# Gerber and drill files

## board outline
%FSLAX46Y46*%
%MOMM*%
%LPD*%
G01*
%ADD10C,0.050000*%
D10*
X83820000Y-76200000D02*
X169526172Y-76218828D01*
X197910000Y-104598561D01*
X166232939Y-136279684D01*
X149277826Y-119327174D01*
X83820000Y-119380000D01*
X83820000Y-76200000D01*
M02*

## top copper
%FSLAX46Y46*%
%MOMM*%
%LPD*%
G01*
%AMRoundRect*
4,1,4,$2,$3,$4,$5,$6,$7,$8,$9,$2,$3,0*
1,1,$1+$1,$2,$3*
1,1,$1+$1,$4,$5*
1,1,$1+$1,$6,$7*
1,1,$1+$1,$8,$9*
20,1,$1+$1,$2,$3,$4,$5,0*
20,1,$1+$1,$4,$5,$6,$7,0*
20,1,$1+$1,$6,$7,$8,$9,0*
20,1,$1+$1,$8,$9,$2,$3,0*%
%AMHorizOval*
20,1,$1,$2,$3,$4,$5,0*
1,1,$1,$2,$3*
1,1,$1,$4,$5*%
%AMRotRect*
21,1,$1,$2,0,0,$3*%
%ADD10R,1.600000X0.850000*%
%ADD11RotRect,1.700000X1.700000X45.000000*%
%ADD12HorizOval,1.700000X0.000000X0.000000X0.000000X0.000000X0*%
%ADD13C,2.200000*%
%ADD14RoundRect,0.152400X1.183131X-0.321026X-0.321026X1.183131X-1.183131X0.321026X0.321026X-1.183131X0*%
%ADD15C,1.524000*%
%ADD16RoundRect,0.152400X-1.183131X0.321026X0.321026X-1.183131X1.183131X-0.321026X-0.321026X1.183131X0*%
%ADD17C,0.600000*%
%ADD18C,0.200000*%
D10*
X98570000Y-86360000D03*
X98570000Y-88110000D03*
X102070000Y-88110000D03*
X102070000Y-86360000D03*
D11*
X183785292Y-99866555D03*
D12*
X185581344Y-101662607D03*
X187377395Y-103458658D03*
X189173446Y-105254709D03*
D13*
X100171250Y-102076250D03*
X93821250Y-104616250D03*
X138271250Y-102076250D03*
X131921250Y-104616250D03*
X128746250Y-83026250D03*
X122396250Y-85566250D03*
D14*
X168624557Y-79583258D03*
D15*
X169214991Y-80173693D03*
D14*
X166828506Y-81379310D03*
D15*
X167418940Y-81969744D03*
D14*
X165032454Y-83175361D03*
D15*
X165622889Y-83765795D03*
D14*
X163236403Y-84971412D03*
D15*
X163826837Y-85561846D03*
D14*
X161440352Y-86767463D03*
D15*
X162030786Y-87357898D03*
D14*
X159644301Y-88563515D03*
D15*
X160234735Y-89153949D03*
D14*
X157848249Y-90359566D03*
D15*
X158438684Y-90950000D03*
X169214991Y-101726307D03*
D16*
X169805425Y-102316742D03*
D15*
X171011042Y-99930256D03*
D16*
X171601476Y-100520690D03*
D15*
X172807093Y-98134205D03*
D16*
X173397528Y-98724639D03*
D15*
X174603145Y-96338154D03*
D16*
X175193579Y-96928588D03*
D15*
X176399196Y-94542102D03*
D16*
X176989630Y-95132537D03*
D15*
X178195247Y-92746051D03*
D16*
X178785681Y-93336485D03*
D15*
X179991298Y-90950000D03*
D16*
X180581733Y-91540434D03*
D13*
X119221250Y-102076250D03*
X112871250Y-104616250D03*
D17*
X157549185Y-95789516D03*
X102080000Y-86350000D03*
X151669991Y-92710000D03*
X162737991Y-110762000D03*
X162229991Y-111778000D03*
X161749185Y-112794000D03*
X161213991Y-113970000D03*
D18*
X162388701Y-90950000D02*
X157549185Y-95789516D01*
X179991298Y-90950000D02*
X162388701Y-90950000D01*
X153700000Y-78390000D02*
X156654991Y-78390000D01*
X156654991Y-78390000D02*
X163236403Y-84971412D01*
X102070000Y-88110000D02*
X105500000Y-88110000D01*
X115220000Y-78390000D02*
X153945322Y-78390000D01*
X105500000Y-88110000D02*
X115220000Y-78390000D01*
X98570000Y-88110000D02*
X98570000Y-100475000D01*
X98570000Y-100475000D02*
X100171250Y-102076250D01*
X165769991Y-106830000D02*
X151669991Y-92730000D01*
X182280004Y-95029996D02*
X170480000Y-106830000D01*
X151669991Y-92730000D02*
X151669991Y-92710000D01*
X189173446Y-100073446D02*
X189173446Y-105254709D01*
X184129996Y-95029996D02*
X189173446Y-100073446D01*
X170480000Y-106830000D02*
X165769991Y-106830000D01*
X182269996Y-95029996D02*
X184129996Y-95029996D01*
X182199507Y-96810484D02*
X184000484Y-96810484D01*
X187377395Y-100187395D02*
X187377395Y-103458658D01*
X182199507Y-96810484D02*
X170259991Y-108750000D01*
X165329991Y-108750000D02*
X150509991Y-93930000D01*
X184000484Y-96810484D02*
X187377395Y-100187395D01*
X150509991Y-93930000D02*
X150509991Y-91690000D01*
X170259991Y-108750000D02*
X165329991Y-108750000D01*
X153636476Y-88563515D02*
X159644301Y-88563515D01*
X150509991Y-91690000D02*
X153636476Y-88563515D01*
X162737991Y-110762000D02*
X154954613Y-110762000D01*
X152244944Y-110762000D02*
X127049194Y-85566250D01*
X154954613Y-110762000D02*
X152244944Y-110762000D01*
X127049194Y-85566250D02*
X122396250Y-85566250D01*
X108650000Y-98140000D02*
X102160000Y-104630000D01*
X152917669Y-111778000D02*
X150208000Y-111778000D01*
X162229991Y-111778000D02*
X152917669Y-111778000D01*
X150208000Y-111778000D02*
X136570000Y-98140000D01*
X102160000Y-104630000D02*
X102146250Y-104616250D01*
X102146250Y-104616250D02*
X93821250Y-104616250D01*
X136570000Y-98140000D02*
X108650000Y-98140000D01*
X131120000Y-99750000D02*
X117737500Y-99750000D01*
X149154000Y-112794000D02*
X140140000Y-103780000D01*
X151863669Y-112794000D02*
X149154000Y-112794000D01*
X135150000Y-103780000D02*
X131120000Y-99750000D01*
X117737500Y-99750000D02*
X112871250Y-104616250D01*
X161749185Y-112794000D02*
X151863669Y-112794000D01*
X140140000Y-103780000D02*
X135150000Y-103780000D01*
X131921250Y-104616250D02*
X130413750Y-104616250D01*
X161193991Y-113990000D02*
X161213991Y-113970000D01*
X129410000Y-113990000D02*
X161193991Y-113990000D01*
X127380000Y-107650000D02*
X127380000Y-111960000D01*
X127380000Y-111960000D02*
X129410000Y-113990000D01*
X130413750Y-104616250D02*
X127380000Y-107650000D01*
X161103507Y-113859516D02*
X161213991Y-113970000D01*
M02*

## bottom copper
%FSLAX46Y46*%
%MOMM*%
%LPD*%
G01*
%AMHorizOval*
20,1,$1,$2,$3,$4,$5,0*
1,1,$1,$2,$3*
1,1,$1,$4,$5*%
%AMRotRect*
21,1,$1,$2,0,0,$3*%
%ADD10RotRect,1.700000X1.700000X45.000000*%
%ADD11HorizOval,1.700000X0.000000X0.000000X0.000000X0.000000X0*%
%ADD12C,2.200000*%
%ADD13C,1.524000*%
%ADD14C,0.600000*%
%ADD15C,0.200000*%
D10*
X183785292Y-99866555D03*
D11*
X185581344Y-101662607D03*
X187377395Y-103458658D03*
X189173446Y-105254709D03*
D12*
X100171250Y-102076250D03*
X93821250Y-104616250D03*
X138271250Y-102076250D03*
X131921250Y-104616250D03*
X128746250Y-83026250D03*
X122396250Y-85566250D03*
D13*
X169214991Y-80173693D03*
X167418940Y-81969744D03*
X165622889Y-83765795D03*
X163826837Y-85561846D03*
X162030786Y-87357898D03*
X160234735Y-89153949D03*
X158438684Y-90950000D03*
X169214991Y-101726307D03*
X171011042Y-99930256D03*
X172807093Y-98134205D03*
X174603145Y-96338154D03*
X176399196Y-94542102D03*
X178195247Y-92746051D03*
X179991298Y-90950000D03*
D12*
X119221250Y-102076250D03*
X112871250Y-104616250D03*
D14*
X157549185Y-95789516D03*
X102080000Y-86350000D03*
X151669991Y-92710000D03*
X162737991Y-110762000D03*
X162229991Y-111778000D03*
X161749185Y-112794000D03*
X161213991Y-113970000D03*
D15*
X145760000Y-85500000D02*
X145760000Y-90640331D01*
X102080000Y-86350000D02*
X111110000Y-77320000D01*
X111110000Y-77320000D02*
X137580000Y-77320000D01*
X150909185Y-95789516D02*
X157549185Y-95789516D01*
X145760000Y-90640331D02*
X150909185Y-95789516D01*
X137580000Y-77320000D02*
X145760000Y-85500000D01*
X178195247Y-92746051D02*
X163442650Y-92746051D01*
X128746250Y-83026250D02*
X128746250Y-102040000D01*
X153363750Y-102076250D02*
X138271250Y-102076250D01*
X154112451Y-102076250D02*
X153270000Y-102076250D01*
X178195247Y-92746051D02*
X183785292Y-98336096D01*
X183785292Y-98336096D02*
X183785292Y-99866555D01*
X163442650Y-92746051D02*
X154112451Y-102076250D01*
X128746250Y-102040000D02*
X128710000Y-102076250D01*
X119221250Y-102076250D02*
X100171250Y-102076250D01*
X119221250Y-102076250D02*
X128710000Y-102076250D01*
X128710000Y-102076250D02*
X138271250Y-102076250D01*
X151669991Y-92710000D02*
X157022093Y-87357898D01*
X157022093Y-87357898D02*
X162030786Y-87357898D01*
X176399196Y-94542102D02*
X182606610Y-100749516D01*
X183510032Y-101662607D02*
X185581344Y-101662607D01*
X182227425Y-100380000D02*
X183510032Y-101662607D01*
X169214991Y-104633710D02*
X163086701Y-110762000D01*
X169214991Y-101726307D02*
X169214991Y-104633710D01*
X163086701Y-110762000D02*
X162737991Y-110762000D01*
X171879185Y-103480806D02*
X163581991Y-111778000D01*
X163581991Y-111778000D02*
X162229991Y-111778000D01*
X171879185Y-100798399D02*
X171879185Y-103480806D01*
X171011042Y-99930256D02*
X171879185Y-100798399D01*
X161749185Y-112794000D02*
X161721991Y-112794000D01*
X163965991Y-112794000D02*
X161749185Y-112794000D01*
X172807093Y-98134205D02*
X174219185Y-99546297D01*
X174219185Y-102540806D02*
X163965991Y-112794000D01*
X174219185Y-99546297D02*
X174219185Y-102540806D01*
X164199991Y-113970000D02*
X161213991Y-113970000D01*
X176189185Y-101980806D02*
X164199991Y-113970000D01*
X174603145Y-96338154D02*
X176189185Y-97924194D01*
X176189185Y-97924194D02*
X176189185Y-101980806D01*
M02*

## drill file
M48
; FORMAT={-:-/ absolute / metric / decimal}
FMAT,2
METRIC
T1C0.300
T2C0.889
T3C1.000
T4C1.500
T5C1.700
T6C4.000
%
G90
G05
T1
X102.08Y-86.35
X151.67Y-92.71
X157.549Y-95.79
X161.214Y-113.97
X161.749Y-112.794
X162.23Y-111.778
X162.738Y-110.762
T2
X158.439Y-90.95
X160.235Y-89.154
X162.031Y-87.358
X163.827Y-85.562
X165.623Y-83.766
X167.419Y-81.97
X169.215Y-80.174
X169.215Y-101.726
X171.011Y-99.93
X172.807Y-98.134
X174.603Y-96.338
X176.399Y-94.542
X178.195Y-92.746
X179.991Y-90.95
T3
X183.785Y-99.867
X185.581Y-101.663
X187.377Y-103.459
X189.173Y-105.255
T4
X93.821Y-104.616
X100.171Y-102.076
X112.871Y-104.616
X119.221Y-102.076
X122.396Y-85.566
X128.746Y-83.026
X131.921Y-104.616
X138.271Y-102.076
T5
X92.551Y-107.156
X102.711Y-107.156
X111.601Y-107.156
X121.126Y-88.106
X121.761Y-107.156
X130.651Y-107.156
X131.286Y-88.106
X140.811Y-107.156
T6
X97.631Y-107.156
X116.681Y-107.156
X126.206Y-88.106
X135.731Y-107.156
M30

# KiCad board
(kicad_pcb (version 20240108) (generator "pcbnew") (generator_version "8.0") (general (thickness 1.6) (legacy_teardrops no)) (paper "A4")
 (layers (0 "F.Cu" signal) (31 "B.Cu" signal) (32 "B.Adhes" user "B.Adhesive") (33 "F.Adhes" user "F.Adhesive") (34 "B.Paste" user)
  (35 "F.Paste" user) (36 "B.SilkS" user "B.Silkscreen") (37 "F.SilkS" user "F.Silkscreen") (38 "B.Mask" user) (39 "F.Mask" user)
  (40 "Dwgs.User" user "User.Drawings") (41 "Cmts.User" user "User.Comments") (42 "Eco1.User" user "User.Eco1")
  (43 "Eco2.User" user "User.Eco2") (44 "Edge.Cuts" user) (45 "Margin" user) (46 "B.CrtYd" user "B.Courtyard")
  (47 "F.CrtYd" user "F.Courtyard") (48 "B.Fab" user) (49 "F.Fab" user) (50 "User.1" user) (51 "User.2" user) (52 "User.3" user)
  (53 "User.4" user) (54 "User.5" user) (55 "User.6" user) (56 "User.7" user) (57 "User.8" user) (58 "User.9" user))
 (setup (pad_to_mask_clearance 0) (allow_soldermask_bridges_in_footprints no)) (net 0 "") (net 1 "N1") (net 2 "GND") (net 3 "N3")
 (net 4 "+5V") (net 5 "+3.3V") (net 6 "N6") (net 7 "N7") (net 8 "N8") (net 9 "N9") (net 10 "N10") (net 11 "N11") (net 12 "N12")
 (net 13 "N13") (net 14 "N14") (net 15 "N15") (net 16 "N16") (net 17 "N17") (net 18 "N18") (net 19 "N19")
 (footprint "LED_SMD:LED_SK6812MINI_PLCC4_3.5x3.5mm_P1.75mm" (layer "F.Cu") (at 100.32 87.235)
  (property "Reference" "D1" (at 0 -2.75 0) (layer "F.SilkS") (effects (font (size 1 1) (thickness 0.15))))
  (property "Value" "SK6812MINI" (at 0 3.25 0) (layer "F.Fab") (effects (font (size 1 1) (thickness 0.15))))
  (pad "1" smd rect (at -1.75 -0.875) (size 1.6 0.85) (layers "F.Cu" "F.Paste" "F.Mask") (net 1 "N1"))
  (pad "2" smd rect (at -1.75 0.875) (size 1.6 0.85) (layers "F.Cu" "F.Paste" "F.Mask") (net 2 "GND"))
  (pad "3" smd rect (at 1.75 0.875) (size 1.6 0.85) (layers "F.Cu" "F.Paste" "F.Mask") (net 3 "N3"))
  (pad "4" smd rect (at 1.75 -0.875) (size 1.6 0.85) (layers "F.Cu" "F.Paste" "F.Mask") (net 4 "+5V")))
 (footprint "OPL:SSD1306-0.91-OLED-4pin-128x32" (layer "F.Cu") (at 156.427331 124.127389 45)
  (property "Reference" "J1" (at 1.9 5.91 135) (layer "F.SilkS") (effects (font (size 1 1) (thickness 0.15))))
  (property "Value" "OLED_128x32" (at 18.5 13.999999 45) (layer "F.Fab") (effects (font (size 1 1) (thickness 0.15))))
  (pad "1" thru_hole rect (at 36.5 2.19 45) (size 1.7 1.7) (drill 1) (layers "*.Cu" "*.Mask") (remove_unused_layers no) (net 2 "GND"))
  (pad "2" thru_hole oval (at 36.5 4.730001 45) (size 1.7 1.7) (drill 1) (layers "*.Cu" "*.Mask") (remove_unused_layers no) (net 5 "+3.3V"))
  (pad "3" thru_hole oval (at 36.5 7.27 45) (size 1.7 1.7) (drill 1) (layers "*.Cu" "*.Mask") (remove_unused_layers no) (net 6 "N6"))
  (pad "4" thru_hole oval (at 36.5 9.81 45) (size 1.7 1.7) (drill 1) (layers "*.Cu" "*.Mask") (remove_unused_layers no) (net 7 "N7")))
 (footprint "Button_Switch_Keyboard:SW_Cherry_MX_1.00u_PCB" (layer "F.Cu") (at 100.17125 102.07625)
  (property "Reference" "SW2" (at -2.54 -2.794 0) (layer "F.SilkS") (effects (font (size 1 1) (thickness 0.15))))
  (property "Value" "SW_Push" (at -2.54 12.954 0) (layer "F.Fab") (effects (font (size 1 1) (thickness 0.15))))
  (pad "" np_thru_hole circle (at -7.62 5.08) (size 1.7 1.7) (drill 1.7) (layers "*.Cu" "*.Mask"))
  (pad "" np_thru_hole circle (at -2.54 5.08) (size 4 4) (drill 4) (layers "*.Cu" "*.Mask"))
  (pad "" np_thru_hole circle (at 2.54 5.08) (size 1.7 1.7) (drill 1.7) (layers "*.Cu" "*.Mask"))
  (pad "1" thru_hole circle (at 0 0) (size 2.2 2.2) (drill 1.5) (layers "*.Cu" "*.Mask") (remove_unused_layers no) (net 2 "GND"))
  (pad "2" thru_hole circle (at -6.35 2.54) (size 2.2 2.2) (drill 1.5) (layers "*.Cu" "*.Mask") (remove_unused_layers no) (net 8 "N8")))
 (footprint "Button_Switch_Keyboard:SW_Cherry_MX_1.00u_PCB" (layer "F.Cu") (at 138.27125 102.07625)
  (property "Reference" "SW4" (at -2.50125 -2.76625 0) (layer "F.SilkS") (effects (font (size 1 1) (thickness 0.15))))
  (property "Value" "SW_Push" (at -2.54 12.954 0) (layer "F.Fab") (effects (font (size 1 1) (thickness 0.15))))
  (pad "" np_thru_hole circle (at -7.62 5.08) (size 1.7 1.7) (drill 1.7) (layers "*.Cu" "*.Mask"))
  (pad "" np_thru_hole circle (at -2.54 5.08) (size 4 4) (drill 4) (layers "*.Cu" "*.Mask"))
  (pad "" np_thru_hole circle (at 2.54 5.08) (size 1.7 1.7) (drill 1.7) (layers "*.Cu" "*.Mask"))
  (pad "1" thru_hole circle (at 0 0) (size 2.2 2.2) (drill 1.5) (layers "*.Cu" "*.Mask") (remove_unused_layers no) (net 2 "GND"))
  (pad "2" thru_hole circle (at -6.35 2.54) (size 2.2 2.2) (drill 1.5) (layers "*.Cu" "*.Mask") (remove_unused_layers no) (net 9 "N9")))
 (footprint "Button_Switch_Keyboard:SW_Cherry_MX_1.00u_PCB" (layer "F.Cu") (at 128.74625 83.02625)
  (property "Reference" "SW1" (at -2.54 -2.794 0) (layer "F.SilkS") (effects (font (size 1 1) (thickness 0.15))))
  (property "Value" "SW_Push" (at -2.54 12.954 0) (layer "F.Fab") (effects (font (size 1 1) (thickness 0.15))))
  (pad "" np_thru_hole circle (at -7.62 5.08) (size 1.7 1.7) (drill 1.7) (layers "*.Cu" "*.Mask"))
  (pad "" np_thru_hole circle (at -2.54 5.08) (size 4 4) (drill 4) (layers "*.Cu" "*.Mask"))
  (pad "" np_thru_hole circle (at 2.54 5.08) (size 1.7 1.7) (drill 1.7) (layers "*.Cu" "*.Mask"))
  (pad "1" thru_hole circle (at 0 0) (size 2.2 2.2) (drill 1.5) (layers "*.Cu" "*.Mask") (remove_unused_layers no) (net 2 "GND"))
  (pad "2" thru_hole circle (at -6.35 2.54) (size 2.2 2.2) (drill 1.5) (layers "*.Cu" "*.Mask") (remove_unused_layers no) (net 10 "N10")))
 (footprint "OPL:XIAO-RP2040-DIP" (layer "F.Cu") (at 169.214991 90.95 -45)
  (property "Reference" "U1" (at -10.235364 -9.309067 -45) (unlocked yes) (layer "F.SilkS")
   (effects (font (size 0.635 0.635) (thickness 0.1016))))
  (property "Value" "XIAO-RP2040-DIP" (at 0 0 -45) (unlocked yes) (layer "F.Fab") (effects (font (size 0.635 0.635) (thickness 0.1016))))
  (pad "1" smd roundrect (at -8.455 -7.62 135) (size 2.432 1.524) (layers "F.Cu" "F.Mask") (roundrect_rratio 0.1) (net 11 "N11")
   (thermal_bridge_angle 45))
  (pad "1" thru_hole circle (at -7.62 -7.62 135) (size 1.524 1.524) (drill 0.889) (layers "*.Cu" "*.Mask") (remove_unused_layers no)
   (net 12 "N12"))
  (pad "2" smd roundrect (at -8.455 -5.08 135) (size 2.432 1.524) (layers "F.Cu" "F.Mask") (roundrect_rratio 0.1) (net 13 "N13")
   (thermal_bridge_angle 45))
  (pad "2" thru_hole circle (at -7.62 -5.08 135) (size 1.524 1.524) (drill 0.889) (layers "*.Cu" "*.Mask") (remove_unused_layers no)
   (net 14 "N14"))
  (pad "3" smd roundrect (at -8.455 -2.54 135) (size 2.432 1.524) (layers "F.Cu" "F.Mask") (roundrect_rratio 0.1) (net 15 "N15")
   (thermal_bridge_angle 45))
  (pad "3" thru_hole circle (at -7.62 -2.54 135) (size 1.524 1.524) (drill 0.889) (layers "*.Cu" "*.Mask") (remove_unused_layers no)
   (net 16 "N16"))
  (pad "4" smd roundrect (at -8.455 0 135) (size 2.432 1.524) (layers "F.Cu" "F.Mask") (roundrect_rratio 0.1) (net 3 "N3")
   (thermal_bridge_angle 45))
  (pad "4" thru_hole circle (at -7.62 0 135) (size 1.524 1.524) (drill 0.889) (layers "*.Cu" "*.Mask") (remove_unused_layers no)
   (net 3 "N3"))
  (pad "5" smd roundrect (at -8.455 2.54 135) (size 2.432 1.524) (layers "F.Cu" "F.Mask") (roundrect_rratio 0.1) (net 7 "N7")
   (thermal_bridge_angle 45))
  (pad "5" thru_hole circle (at -7.62 2.54 135) (size 1.524 1.524) (drill 0.889) (layers "*.Cu" "*.Mask") (remove_unused_layers no)
   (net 7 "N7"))
  (pad "6" smd roundrect (at -8.455 5.08 135) (size 2.432 1.524) (layers "F.Cu" "F.Mask") (roundrect_rratio 0.1) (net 6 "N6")
   (thermal_bridge_angle 45))
  (pad "6" thru_hole circle (at -7.62 5.08 135) (size 1.524 1.524) (drill 0.889) (layers "*.Cu" "*.Mask") (remove_unused_layers no)
   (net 6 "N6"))
  (pad "7" smd roundrect (at -8.455 7.62 135) (size 2.432 1.524) (layers "F.Cu" "F.Mask") (roundrect_rratio 0.1) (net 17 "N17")
   (thermal_bridge_angle 45))
  (pad "7" thru_hole circle (at -7.62 7.62 135) (size 1.524 1.524) (drill 0.889) (layers "*.Cu" "*.Mask") (remove_unused_layers no)
   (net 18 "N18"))
  (pad "8" thru_hole circle (at 7.62 7.62 315) (size 1.524 1.524) (drill 0.889) (layers "*.Cu" "*.Mask") (remove_unused_layers no)
   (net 10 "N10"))
  (pad "8" smd roundrect (at 8.455 7.62 315) (size 2.432 1.524) (layers "F.Cu" "F.Mask") (roundrect_rratio 0.1) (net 10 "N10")
   (thermal_bridge_angle 45))
  (pad "9" thru_hole circle (at 7.62 5.08 315) (size 1.524 1.524) (drill 0.889) (layers "*.Cu" "*.Mask") (remove_unused_layers no)
   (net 8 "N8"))
  (pad "9" smd roundrect (at 8.455 5.08 315) (size 2.432 1.524) (layers "F.Cu" "F.Mask") (roundrect_rratio 0.1) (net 8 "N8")
   (thermal_bridge_angle 45))
  (pad "10" thru_hole circle (at 7.62 2.54 315) (size 1.524 1.524) (drill 0.889) (layers "*.Cu" "*.Mask") (remove_unused_layers no)
   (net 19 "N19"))
  (pad "10" smd roundrect (at 8.455 2.54 315) (size 2.432 1.524) (layers "F.Cu" "F.Mask") (roundrect_rratio 0.1) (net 19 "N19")
   (thermal_bridge_angle 45))
  (pad "11" thru_hole circle (at 7.62 0 315) (size 1.524 1.524) (drill 0.889) (layers "*.Cu" "*.Mask") (remove_unused_layers no)
   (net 9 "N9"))
  (pad "11" smd roundrect (at 8.455 0 315) (size 2.432 1.524) (layers "F.Cu" "F.Mask") (roundrect_rratio 0.1) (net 9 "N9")
   (thermal_bridge_angle 45))
  (pad "12" thru_hole circle (at 7.62 -2.54 315) (size 1.524 1.524) (drill 0.889) (layers "*.Cu" "*.Mask") (remove_unused_layers no)
   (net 5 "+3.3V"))
  (pad "12" smd roundrect (at 8.455 -2.54 315) (size 2.432 1.524) (layers "F.Cu" "F.Mask") (roundrect_rratio 0.1) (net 5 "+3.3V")
   (thermal_bridge_angle 45))
  (pad "13" thru_hole circle (at 7.62 -5.08 315) (size 1.524 1.524) (drill 0.889) (layers "*.Cu" "*.Mask") (remove_unused_layers no)
   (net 2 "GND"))
  (pad "13" smd roundrect (at 8.455 -5.08 315) (size 2.432 1.524) (layers "F.Cu" "F.Mask") (roundrect_rratio 0.1) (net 2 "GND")
   (thermal_bridge_angle 45))
  (pad "14" thru_hole circle (at 7.62 -7.62 315) (size 1.524 1.524) (drill 0.889) (layers "*.Cu" "*.Mask") (remove_unused_layers no)
   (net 4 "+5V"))
  (pad "14" smd roundrect (at 8.455 -7.62 315) (size 2.432 1.524) (layers "F.Cu" "F.Mask") (roundrect_rratio 0.1) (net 4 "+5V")
   (thermal_bridge_angle 45)))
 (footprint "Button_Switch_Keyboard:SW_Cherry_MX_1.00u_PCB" (layer "F.Cu") (at 119.22125 102.07625)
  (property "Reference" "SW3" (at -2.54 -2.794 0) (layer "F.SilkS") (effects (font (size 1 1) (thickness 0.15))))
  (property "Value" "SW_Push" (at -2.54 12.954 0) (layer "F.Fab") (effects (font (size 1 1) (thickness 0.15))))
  (pad "" np_thru_hole circle (at -7.62 5.08) (size 1.7 1.7) (drill 1.7) (layers "*.Cu" "*.Mask"))
  (pad "" np_thru_hole circle (at -2.54 5.08) (size 4 4) (drill 4) (layers "*.Cu" "*.Mask"))
  (pad "" np_thru_hole circle (at 2.54 5.08) (size 1.7 1.7) (drill 1.7) (layers "*.Cu" "*.Mask"))
  (pad "1" thru_hole circle (at 0 0) (size 2.2 2.2) (drill 1.5) (layers "*.Cu" "*.Mask") (remove_unused_layers no) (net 2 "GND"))
  (pad "2" thru_hole circle (at -6.35 2.54) (size 2.2 2.2) (drill 1.5) (layers "*.Cu" "*.Mask") (remove_unused_layers no) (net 19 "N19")))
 (gr_poly
  (pts (xy 83.82 76.2) (xy 169.526172 76.218828) (xy 197.91 104.598561) (xy 166.232939 136.279684) (xy 149.277826 119.327174)
   (xy 83.82 119.38))
  (stroke (width 0.05) (type solid)) (fill none) (layer "Edge.Cuts"))
 (segment (start 162.388701 90.95) (end 157.549185 95.789516) (width 0.2) (layer "F.Cu") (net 4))
 (segment (start 179.991298 90.95) (end 162.388701 90.95) (width 0.2) (layer "F.Cu") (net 4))
 (via (at 157.549185 95.789516) (size 0.6) (drill 0.3) (layers "F.Cu" "B.Cu") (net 4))
 (via (at 102.08 86.35) (size 0.6) (drill 0.3) (layers "F.Cu" "B.Cu") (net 4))
 (segment (start 145.76 85.5) (end 145.76 90.640331) (width 0.2) (layer "B.Cu") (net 4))
 (segment (start 102.08 86.35) (end 111.11 77.32) (width 0.2) (layer "B.Cu") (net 4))
 (segment (start 111.11 77.32) (end 137.58 77.32) (width 0.2) (layer "B.Cu") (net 4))
 (segment (start 150.909185 95.789516) (end 157.549185 95.789516) (width 0.2) (layer "B.Cu") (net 4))
 (segment (start 145.76 90.640331) (end 150.909185 95.789516) (width 0.2) (layer "B.Cu") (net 4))
 (segment (start 137.58 77.32) (end 145.76 85.5) (width 0.2) (layer "B.Cu") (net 4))
 (segment (start 153.7 78.39) (end 156.654991 78.39) (width 0.2) (layer "F.Cu") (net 3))
 (segment (start 156.654991 78.39) (end 163.236403 84.971412) (width 0.2) (layer "F.Cu") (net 3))
 (segment (start 102.07 88.11) (end 105.5 88.11) (width 0.2) (layer "F.Cu") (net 3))
 (segment (start 115.22 78.39) (end 153.945322 78.39) (width 0.2) (layer "F.Cu") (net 3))
 (segment (start 105.5 88.11) (end 115.22 78.39) (width 0.2) (layer "F.Cu") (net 3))
 (segment (start 98.57 88.11) (end 98.57 100.475) (width 0.2) (layer "F.Cu") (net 2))
 (segment (start 98.57 100.475) (end 100.17125 102.07625) (width 0.2) (layer "F.Cu") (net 2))
 (segment (start 178.195247 92.746051) (end 163.44265 92.746051) (width 0.2) (layer "B.Cu") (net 2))
 (segment (start 128.74625 83.02625) (end 128.74625 102.04) (width 0.2) (layer "B.Cu") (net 2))
 (segment (start 153.36375 102.07625) (end 138.27125 102.07625) (width 0.2) (layer "B.Cu") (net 2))
 (segment (start 154.112451 102.07625) (end 153.27 102.07625) (width 0.2) (layer "B.Cu") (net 2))
 (segment (start 178.195247 92.746051) (end 183.785292 98.336096) (width 0.2) (layer "B.Cu") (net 2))
 (segment (start 183.785292 98.336096) (end 183.785292 99.866555) (width 0.2) (layer "B.Cu") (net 2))
 (segment (start 163.44265 92.746051) (end 154.112451 102.07625) (width 0.2) (layer "B.Cu") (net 2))
 (segment (start 128.74625 102.04) (end 128.71 102.07625) (width 0.2) (layer "B.Cu") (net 2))
 (segment (start 119.22125 102.07625) (end 100.17125 102.07625) (width 0.2) (layer "B.Cu") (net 2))
 (segment (start 119.22125 102.07625) (end 128.71 102.07625) (width 0.2) (layer "B.Cu") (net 2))
 (segment (start 128.71 102.07625) (end 138.27125 102.07625) (width 0.2) (layer "B.Cu") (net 2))
 (segment (start 165.769991 106.83) (end 151.669991 92.73) (width 0.2) (layer "F.Cu") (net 7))
 (segment (start 182.280004 95.029996) (end 170.48 106.83) (width 0.2) (layer "F.Cu") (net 7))
 (segment (start 151.669991 92.73) (end 151.669991 92.71) (width 0.2) (layer "F.Cu") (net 7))
 (segment (start 189.173446 100.073446) (end 189.173446 105.254709) (width 0.2) (layer "F.Cu") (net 7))
 (segment (start 184.129996 95.029996) (end 189.173446 100.073446) (width 0.2) (layer "F.Cu") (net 7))
 (segment (start 170.48 106.83) (end 165.769991 106.83) (width 0.2) (layer "F.Cu") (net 7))
 (segment (start 182.269996 95.029996) (end 184.129996 95.029996) (width 0.2) (layer "F.Cu") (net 7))
 (via (at 151.669991 92.71) (size 0.6) (drill 0.3) (layers "F.Cu" "B.Cu") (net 7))
 (segment (start 151.669991 92.71) (end 157.022093 87.357898) (width 0.2) (layer "B.Cu") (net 7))
 (segment (start 157.022093 87.357898) (end 162.030786 87.357898) (width 0.2) (layer "B.Cu") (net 7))
 (segment (start 182.199507 96.810484) (end 184.000484 96.810484) (width 0.2) (layer "F.Cu") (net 6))
 (segment (start 187.377395 100.187395) (end 187.377395 103.458658) (width 0.2) (layer "F.Cu") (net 6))
 (segment (start 182.199507 96.810484) (end 170.259991 108.75) (width 0.2) (layer "F.Cu") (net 6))
 (segment (start 165.329991 108.75) (end 150.509991 93.93) (width 0.2) (layer "F.Cu") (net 6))
 (segment (start 184.000484 96.810484) (end 187.377395 100.187395) (width 0.2) (layer "F.Cu") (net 6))
 (segment (start 150.509991 93.93) (end 150.509991 91.69) (width 0.2) (layer "F.Cu") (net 6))
 (segment (start 170.259991 108.75) (end 165.329991 108.75) (width 0.2) (layer "F.Cu") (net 6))
 (segment (start 153.636476 88.563515) (end 159.644301 88.563515) (width 0.2) (layer "F.Cu") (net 6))
 (segment (start 150.509991 91.69) (end 153.636476 88.563515) (width 0.2) (layer "F.Cu") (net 6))
 (segment (start 176.399196 94.542102) (end 182.60661 100.749516) (width 0.2) (layer "B.Cu") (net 5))
 (segment (start 183.510032 101.662607) (end 185.581344 101.662607) (width 0.2) (layer "B.Cu") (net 5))
 (segment (start 182.227425 100.38) (end 183.510032 101.662607) (width 0.2) (layer "B.Cu") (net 5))
 (segment (start 162.737991 110.762) (end 154.954613 110.762) (width 0.2) (layer "F.Cu") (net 10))
 (segment (start 152.244944 110.762) (end 127.049194 85.56625) (width 0.2) (layer "F.Cu") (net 10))
 (segment (start 154.954613 110.762) (end 152.244944 110.762) (width 0.2) (layer "F.Cu") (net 10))
 (segment (start 127.049194 85.56625) (end 122.39625 85.56625) (width 0.2) (layer "F.Cu") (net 10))
 (via (at 162.737991 110.762) (size 0.6) (drill 0.3) (layers "F.Cu" "B.Cu") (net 10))
 (segment (start 169.214991 104.63371) (end 163.086701 110.762) (width 0.2) (layer "B.Cu") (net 10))
 (segment (start 169.214991 101.726307) (end 169.214991 104.63371) (width 0.2) (layer "B.Cu") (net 10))
 (segment (start 163.086701 110.762) (end 162.737991 110.762) (width 0.2) (layer "B.Cu") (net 10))
 (segment (start 108.65 98.14) (end 102.16 104.63) (width 0.2) (layer "F.Cu") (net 8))
 (segment (start 152.917669 111.778) (end 150.208 111.778) (width 0.2) (layer "F.Cu") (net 8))
 (segment (start 162.229991 111.778) (end 152.917669 111.778) (width 0.2) (layer "F.Cu") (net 8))
 (segment (start 150.208 111.778) (end 136.57 98.14) (width 0.2) (layer "F.Cu") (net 8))
 (segment (start 102.16 104.63) (end 102.14625 104.61625) (width 0.2) (layer "F.Cu") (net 8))
 (segment (start 102.14625 104.61625) (end 93.82125 104.61625) (width 0.2) (layer "F.Cu") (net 8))
 (segment (start 136.57 98.14) (end 108.65 98.14) (width 0.2) (layer "F.Cu") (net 8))
 (via (at 162.229991 111.778) (size 0.6) (drill 0.3) (layers "F.Cu" "B.Cu") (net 8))
 (segment (start 171.879185 103.480806) (end 163.581991 111.778) (width 0.2) (layer "B.Cu") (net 8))
 (segment (start 163.581991 111.778) (end 162.229991 111.778) (width 0.2) (layer "B.Cu") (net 8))
 (segment (start 171.879185 100.798399) (end 171.879185 103.480806) (width 0.2) (layer "B.Cu") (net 8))
 (segment (start 171.011042 99.930256) (end 171.879185 100.798399) (width 0.2) (layer "B.Cu") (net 8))
 (segment (start 131.12 99.75) (end 117.7375 99.75) (width 0.2) (layer "F.Cu") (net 19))
 (segment (start 149.154 112.794) (end 140.14 103.78) (width 0.2) (layer "F.Cu") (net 19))
 (segment (start 151.863669 112.794) (end 149.154 112.794) (width 0.2) (layer "F.Cu") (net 19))
 (segment (start 135.15 103.78) (end 131.12 99.75) (width 0.2) (layer "F.Cu") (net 19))
 (segment (start 117.7375 99.75) (end 112.87125 104.61625) (width 0.2) (layer "F.Cu") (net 19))
 (segment (start 161.749185 112.794) (end 151.863669 112.794) (width 0.2) (layer "F.Cu") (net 19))
 (segment (start 140.14 103.78) (end 135.15 103.78) (width 0.2) (layer "F.Cu") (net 19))
 (via (at 161.749185 112.794) (size 0.6) (drill 0.3) (layers "F.Cu" "B.Cu") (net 19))
 (segment (start 161.749185 112.794) (end 161.721991 112.794) (width 0.2) (layer "B.Cu") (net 19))
 (segment (start 163.965991 112.794) (end 161.749185 112.794) (width 0.2) (layer "B.Cu") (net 19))
 (segment (start 172.807093 98.134205) (end 174.219185 99.546297) (width 0.2) (layer "B.Cu") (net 19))
 (segment (start 174.219185 102.540806) (end 163.965991 112.794) (width 0.2) (layer "B.Cu") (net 19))
 (segment (start 174.219185 99.546297) (end 174.219185 102.540806) (width 0.2) (layer "B.Cu") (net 19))
 (segment (start 131.92125 104.61625) (end 130.41375 104.61625) (width 0.2) (layer "F.Cu") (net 9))
 (segment (start 161.193991 113.99) (end 161.213991 113.97) (width 0.2) (layer "F.Cu") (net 9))
 (segment (start 129.41 113.99) (end 161.193991 113.99) (width 0.2) (layer "F.Cu") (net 9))
 (segment (start 127.38 107.65) (end 127.38 111.96) (width 0.2) (layer "F.Cu") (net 9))
 (segment (start 127.38 111.96) (end 129.41 113.99) (width 0.2) (layer "F.Cu") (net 9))
 (segment (start 130.41375 104.61625) (end 127.38 107.65) (width 0.2) (layer "F.Cu") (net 9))
 (segment (start 161.103507 113.859516) (end 161.213991 113.97) (width 0.2) (layer "F.Cu") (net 9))
 (via (at 161.213991 113.97) (size 0.6) (drill 0.3) (layers "F.Cu" "B.Cu") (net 9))
 (segment (start 164.199991 113.97) (end 161.213991 113.97) (width 0.2) (layer "B.Cu") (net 9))
 (segment (start 176.189185 101.980806) (end 164.199991 113.97) (width 0.2) (layer "B.Cu") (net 9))
 (segment (start 174.603145 96.338154) (end 176.189185 97.924194) (width 0.2) (layer "B.Cu") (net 9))
 (segment (start 176.189185 97.924194) (end 176.189185 101.980806) (width 0.2) (layer "B.Cu") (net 9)))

